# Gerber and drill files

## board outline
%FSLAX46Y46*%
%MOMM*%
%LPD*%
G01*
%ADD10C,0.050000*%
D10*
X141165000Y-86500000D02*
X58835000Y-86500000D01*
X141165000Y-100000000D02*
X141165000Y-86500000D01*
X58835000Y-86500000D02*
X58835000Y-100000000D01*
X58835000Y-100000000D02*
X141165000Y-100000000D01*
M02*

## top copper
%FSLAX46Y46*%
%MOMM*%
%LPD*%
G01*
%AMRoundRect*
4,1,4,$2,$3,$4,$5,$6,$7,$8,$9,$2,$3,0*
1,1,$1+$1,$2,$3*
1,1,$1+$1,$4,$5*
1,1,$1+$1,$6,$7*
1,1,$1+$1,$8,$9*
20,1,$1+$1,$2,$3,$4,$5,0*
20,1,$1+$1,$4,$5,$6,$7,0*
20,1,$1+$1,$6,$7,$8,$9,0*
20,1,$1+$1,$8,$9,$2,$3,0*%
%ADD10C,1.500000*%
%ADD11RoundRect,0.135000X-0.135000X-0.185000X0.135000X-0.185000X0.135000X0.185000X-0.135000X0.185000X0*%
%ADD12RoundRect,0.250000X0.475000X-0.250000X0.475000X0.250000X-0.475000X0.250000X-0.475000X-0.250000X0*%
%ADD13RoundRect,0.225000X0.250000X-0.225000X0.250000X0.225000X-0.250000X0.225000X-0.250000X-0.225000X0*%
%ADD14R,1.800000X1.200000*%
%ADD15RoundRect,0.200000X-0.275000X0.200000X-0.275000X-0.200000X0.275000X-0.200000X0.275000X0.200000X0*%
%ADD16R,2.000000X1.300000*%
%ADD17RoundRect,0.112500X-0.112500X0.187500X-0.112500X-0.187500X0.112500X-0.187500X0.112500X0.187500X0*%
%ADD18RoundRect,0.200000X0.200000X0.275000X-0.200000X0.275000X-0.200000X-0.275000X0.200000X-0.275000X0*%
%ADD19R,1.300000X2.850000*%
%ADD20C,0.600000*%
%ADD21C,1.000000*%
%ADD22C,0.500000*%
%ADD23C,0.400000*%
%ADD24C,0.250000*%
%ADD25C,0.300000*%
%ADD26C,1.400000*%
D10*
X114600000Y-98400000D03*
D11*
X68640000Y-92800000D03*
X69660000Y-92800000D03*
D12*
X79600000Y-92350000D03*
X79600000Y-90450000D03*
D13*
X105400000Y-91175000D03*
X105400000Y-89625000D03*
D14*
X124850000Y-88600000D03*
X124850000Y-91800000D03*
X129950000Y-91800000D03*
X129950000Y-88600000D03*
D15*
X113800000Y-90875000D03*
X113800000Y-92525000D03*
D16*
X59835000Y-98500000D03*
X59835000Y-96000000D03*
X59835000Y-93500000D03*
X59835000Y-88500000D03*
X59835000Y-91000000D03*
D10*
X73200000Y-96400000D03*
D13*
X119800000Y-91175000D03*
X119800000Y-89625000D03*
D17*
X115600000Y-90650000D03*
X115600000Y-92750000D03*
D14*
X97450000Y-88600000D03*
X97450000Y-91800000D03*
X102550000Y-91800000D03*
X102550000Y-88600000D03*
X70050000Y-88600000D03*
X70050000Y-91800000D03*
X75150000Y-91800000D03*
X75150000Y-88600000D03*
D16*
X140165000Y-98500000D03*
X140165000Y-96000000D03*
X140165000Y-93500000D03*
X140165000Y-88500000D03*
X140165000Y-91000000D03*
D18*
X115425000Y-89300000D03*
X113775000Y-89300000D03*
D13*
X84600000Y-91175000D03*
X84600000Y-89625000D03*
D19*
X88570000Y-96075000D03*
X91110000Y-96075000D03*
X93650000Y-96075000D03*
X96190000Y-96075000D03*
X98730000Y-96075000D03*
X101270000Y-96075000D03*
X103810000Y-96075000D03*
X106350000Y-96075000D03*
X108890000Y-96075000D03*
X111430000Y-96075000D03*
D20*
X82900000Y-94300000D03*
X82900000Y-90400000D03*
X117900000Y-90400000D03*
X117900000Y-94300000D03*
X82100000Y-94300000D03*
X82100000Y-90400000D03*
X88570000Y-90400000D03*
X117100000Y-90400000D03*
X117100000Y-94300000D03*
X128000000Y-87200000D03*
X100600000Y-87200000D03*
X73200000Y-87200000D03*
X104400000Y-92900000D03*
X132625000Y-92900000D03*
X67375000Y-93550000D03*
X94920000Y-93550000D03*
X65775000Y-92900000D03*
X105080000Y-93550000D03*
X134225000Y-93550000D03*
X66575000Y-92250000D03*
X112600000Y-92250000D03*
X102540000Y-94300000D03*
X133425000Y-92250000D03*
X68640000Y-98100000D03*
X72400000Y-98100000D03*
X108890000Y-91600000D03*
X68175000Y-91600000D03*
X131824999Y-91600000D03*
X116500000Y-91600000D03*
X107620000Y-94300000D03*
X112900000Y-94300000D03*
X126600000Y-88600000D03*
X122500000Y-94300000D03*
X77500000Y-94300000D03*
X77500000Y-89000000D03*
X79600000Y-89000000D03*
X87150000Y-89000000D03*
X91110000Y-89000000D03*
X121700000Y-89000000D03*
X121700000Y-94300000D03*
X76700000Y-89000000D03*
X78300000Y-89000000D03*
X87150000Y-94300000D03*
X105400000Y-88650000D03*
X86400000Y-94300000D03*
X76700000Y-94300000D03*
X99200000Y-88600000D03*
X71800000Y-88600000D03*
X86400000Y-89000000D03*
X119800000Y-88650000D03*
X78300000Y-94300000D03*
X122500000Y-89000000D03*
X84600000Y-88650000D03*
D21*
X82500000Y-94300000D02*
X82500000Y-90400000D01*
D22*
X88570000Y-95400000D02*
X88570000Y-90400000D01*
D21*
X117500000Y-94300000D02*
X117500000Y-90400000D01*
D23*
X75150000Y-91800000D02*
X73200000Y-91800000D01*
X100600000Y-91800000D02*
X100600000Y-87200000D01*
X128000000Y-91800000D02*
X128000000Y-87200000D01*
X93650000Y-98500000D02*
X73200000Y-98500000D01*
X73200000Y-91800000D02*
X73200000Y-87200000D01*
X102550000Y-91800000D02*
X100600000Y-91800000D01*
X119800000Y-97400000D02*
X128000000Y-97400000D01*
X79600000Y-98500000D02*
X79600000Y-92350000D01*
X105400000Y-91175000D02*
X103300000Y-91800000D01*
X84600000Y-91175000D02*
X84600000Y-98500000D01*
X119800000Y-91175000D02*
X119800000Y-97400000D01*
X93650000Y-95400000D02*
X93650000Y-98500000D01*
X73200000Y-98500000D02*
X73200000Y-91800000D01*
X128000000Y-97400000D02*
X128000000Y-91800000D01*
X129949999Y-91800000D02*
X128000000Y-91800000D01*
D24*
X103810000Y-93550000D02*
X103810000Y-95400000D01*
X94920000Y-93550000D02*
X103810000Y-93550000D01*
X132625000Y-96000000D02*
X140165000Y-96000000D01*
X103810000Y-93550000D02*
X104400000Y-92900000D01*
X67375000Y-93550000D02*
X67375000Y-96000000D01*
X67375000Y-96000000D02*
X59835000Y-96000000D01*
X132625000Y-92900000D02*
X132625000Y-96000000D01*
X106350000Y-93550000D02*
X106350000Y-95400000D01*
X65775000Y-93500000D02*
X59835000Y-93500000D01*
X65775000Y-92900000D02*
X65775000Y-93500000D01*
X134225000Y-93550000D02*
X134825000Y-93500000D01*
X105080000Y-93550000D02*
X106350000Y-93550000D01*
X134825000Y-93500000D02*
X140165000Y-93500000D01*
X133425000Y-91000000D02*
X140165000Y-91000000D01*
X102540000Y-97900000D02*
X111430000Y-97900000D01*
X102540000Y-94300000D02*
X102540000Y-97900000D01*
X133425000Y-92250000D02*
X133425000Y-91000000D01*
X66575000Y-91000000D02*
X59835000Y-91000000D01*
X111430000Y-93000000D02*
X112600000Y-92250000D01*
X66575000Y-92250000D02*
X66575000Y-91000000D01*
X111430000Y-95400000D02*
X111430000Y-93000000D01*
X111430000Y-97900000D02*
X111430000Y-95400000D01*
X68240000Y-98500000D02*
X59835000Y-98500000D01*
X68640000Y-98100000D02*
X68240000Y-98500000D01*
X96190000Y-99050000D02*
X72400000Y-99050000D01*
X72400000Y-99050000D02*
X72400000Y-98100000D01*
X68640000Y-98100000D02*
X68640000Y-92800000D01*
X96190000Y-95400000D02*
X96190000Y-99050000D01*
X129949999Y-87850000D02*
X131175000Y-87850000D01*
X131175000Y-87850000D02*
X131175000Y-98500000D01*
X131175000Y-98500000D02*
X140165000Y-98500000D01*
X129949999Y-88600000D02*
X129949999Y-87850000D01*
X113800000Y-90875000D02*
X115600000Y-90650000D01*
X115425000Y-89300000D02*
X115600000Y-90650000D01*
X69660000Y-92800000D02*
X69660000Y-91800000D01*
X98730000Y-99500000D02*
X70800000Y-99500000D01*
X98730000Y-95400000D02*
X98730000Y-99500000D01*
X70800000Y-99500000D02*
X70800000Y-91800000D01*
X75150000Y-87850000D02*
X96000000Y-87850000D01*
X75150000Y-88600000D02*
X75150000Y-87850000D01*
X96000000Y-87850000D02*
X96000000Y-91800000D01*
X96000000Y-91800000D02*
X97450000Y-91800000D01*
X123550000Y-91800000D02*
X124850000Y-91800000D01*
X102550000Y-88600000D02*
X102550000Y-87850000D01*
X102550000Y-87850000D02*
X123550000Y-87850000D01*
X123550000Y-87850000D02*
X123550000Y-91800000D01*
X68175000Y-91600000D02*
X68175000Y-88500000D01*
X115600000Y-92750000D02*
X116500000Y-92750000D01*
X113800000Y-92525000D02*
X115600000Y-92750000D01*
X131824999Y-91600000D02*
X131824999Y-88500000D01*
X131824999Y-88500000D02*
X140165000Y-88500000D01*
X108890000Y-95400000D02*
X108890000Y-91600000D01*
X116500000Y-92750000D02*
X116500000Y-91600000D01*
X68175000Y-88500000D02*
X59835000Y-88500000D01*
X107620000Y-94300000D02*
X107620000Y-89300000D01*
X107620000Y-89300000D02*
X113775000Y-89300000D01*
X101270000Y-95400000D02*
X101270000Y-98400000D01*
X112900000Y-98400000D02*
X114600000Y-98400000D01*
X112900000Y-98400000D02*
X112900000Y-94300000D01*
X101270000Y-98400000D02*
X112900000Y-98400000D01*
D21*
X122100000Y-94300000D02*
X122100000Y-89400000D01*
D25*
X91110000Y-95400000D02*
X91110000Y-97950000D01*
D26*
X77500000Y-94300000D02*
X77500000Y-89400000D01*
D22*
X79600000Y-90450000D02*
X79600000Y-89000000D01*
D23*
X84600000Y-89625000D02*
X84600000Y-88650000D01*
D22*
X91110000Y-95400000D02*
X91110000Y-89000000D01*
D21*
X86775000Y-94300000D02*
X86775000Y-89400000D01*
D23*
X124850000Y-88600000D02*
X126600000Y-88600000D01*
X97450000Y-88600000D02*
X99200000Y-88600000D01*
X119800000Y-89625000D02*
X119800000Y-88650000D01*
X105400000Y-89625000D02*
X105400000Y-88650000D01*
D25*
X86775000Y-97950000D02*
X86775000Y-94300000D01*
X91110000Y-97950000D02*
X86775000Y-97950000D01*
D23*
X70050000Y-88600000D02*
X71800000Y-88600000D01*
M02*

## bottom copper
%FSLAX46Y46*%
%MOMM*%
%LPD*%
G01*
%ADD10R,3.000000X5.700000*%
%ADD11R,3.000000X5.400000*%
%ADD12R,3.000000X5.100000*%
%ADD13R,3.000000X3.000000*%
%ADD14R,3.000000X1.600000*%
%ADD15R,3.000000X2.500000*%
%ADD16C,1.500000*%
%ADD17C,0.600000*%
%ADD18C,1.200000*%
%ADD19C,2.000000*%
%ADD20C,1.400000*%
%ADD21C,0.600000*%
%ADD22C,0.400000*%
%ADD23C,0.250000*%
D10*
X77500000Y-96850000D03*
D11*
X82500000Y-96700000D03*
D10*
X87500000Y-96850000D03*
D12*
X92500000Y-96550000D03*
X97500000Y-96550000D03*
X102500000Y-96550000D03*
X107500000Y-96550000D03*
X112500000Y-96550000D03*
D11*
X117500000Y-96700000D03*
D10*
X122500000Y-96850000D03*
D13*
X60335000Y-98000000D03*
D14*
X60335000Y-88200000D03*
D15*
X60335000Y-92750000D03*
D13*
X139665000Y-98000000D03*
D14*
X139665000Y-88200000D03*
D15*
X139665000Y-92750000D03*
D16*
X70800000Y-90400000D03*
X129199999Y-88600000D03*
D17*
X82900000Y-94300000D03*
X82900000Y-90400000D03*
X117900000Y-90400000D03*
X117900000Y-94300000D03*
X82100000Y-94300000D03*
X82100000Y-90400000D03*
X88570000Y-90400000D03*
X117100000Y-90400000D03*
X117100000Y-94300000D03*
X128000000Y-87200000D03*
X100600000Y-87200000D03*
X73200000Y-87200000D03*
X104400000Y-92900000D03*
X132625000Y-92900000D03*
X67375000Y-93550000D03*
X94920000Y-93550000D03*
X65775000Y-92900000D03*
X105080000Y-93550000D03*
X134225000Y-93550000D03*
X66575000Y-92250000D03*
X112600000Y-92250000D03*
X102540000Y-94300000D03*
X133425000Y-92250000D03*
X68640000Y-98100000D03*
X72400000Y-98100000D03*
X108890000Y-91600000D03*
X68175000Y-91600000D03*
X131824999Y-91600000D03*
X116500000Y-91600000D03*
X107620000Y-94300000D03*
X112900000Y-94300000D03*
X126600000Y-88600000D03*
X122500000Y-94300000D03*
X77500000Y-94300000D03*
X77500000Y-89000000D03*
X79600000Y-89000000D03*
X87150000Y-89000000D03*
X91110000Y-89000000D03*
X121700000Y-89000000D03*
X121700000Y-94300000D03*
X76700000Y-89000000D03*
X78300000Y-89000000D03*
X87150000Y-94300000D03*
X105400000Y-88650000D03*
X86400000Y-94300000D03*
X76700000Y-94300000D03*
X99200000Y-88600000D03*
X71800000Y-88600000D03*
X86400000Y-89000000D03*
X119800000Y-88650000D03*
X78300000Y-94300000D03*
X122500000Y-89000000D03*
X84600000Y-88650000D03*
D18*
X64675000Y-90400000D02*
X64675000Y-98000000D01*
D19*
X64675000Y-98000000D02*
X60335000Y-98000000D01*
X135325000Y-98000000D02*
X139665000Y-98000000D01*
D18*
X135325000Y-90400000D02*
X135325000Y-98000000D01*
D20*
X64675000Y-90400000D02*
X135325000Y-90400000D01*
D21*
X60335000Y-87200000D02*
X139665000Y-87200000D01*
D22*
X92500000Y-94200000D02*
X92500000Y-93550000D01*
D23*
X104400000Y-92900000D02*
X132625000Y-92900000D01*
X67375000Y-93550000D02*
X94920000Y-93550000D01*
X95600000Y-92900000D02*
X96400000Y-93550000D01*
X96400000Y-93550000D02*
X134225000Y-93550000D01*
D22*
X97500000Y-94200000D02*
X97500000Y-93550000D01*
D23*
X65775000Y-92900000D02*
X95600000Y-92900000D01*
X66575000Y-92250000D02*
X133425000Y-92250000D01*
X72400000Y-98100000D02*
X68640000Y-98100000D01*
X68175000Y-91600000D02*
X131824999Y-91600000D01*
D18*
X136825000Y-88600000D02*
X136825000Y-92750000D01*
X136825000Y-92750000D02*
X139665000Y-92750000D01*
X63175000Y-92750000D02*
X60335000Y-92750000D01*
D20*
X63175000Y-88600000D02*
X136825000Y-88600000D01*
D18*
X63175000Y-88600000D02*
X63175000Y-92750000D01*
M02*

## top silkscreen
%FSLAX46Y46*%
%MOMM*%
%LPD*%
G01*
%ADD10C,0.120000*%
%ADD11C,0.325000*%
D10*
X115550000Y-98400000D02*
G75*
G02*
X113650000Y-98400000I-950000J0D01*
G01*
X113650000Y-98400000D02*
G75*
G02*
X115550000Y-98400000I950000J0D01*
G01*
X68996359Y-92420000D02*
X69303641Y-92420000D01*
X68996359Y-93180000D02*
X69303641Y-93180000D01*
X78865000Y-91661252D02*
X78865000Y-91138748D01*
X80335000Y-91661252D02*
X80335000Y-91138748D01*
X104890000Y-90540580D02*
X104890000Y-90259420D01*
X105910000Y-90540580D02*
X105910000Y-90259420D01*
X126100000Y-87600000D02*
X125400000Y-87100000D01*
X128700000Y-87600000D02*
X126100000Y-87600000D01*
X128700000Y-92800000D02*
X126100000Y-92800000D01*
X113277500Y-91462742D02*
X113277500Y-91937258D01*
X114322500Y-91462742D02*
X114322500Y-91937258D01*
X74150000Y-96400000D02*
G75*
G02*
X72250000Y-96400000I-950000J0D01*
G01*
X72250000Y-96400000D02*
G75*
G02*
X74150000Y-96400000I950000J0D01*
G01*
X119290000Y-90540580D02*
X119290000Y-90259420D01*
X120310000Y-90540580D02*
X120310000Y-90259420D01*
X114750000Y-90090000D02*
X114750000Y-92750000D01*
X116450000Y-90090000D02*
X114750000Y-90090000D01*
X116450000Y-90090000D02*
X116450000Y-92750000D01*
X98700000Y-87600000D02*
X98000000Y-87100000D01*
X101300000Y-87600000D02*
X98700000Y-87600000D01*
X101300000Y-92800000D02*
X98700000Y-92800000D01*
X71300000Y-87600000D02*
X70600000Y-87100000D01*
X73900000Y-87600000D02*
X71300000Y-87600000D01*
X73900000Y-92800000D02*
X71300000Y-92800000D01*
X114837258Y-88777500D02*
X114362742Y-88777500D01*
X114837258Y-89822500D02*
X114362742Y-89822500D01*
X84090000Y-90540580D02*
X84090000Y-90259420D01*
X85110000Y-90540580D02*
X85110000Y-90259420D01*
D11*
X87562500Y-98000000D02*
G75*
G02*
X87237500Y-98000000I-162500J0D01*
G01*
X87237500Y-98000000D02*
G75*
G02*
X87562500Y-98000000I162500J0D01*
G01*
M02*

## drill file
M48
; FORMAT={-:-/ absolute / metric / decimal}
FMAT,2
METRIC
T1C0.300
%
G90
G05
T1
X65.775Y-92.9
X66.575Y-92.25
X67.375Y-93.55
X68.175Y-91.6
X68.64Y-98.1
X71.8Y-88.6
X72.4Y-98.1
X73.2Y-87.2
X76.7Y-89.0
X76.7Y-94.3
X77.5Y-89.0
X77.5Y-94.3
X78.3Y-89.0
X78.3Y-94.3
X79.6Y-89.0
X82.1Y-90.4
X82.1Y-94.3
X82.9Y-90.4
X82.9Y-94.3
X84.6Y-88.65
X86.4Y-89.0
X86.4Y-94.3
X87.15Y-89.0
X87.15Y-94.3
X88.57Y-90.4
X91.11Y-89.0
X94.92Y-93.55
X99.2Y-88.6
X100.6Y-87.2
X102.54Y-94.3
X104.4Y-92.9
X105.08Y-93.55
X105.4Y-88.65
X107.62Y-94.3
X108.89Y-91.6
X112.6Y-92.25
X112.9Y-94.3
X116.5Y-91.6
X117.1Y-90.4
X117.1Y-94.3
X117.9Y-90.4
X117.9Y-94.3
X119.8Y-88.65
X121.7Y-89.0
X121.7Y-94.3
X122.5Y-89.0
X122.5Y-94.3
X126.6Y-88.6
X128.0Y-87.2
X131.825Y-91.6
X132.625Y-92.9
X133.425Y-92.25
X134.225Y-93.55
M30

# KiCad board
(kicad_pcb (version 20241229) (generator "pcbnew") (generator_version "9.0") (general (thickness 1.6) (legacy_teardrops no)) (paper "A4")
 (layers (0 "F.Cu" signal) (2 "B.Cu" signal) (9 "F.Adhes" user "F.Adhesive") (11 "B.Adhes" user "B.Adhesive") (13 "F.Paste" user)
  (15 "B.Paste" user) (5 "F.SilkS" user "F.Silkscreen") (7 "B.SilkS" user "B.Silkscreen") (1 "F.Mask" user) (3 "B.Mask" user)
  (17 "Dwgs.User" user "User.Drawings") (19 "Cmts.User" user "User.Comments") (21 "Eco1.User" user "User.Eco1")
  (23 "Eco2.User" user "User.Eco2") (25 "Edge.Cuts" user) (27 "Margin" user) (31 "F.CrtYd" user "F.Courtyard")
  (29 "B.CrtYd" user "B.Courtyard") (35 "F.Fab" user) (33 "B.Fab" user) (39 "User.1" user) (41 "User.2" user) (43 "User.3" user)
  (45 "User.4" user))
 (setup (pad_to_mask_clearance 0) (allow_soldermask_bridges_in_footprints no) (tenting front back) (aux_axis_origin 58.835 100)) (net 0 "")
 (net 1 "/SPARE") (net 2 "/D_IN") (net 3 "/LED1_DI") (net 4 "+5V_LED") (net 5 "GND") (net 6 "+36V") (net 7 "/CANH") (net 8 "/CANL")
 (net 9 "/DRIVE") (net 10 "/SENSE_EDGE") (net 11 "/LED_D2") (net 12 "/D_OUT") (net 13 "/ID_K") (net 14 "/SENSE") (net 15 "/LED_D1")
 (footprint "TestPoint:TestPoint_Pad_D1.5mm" (layer "F.Cu") (at 114.6 98.4)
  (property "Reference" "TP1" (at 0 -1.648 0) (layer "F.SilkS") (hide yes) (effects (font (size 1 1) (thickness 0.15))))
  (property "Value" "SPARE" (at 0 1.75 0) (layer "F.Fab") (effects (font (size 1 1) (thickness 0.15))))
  (fp_circle (center 0 0) (end 0 0.95) (stroke (width 0.12) (type solid)) (fill no) (layer "F.SilkS"))
  (pad "1" smd circle (at 0 0) (size 1.5 1.5) (layers "F.Cu" "F.Mask") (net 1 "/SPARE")))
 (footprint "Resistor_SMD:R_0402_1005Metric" (layer "F.Cu") (at 69.15 92.8)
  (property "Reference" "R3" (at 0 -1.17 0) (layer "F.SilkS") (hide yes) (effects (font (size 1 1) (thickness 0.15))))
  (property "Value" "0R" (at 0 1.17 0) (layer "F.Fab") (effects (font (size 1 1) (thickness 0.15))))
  (fp_line (start -0.153641 -0.38) (end 0.153641 -0.38) (stroke (width 0.12) (type solid)) (layer "F.SilkS"))
  (fp_line (start -0.153641 0.38) (end 0.153641 0.38) (stroke (width 0.12) (type solid)) (layer "F.SilkS"))
  (pad "1" smd roundrect (at -0.51 0) (size 0.54 0.64) (layers "F.Cu" "F.Mask" "F.Paste") (roundrect_rratio 0.25) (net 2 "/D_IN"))
  (pad "2" smd roundrect (at 0.51 0) (size 0.54 0.64) (layers "F.Cu" "F.Mask" "F.Paste") (roundrect_rratio 0.25) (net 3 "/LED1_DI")))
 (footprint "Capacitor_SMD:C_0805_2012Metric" (layer "F.Cu") (at 79.6 91.4 90)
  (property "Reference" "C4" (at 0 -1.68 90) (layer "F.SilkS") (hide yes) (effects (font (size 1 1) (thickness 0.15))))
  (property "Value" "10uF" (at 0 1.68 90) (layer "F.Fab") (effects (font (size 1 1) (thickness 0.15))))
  (fp_line (start -0.261252 -0.735) (end 0.261252 -0.735) (stroke (width 0.12) (type solid)) (layer "F.SilkS"))
  (fp_line (start -0.261252 0.735) (end 0.261252 0.735) (stroke (width 0.12) (type solid)) (layer "F.SilkS"))
  (pad "1" smd roundrect (at -0.95 0 90) (size 1 1.45) (layers "F.Cu" "F.Mask" "F.Paste") (roundrect_rratio 0.25) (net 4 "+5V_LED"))
  (pad "2" smd roundrect (at 0.95 0 90) (size 1 1.45) (layers "F.Cu" "F.Mask" "F.Paste") (roundrect_rratio 0.25) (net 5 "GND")))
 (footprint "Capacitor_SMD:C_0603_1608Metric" (layer "F.Cu") (at 105.4 90.4 90)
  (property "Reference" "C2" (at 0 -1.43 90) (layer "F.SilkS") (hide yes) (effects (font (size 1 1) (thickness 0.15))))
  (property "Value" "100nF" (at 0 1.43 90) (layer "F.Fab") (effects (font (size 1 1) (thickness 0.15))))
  (fp_line (start -0.14058 -0.51) (end 0.14058 -0.51) (stroke (width 0.12) (type solid)) (layer "F.SilkS"))
  (fp_line (start -0.14058 0.51) (end 0.14058 0.51) (stroke (width 0.12) (type solid)) (layer "F.SilkS"))
  (pad "1" smd roundrect (at -0.775 0 90) (size 0.9 0.95) (layers "F.Cu" "F.Mask" "F.Paste") (roundrect_rratio 0.25) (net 4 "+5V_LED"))
  (pad "2" smd roundrect (at 0.775 0 90) (size 0.9 0.95) (layers "F.Cu" "F.Mask" "F.Paste") (roundrect_rratio 0.25) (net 5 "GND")))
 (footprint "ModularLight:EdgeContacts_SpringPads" (layer "F.Cu") (at 100 100)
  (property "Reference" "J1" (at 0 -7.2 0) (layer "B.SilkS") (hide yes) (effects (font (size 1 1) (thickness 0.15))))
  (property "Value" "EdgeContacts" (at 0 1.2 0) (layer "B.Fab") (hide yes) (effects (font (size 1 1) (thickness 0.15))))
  (pad "X1" smd rect (at -22.5 -3.15) (size 3 5.7) (layers "B.Cu" "B.Mask") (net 5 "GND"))
  (pad "X2" smd rect (at -17.5 -3.3) (size 3 5.4) (layers "B.Cu" "B.Mask") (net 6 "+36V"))
  (pad "X3" smd rect (at -12.5 -3.15) (size 3 5.7) (layers "B.Cu" "B.Mask") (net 5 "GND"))
  (pad "X4" smd rect (at -7.5 -3.45) (size 3 5.1) (layers "B.Cu" "B.Mask") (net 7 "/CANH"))
  (pad "X5" smd rect (at -2.5 -3.45) (size 3 5.1) (layers "B.Cu" "B.Mask") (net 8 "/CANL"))
  (pad "X6" smd rect (at 2.5 -3.45) (size 3 5.1) (layers "B.Cu" "B.Mask") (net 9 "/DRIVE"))
  (pad "X7" smd rect (at 7.5 -3.45) (size 3 5.1) (layers "B.Cu" "B.Mask") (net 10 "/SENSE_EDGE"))
  (pad "X8" smd rect (at 12.5 -3.45) (size 3 5.1) (layers "B.Cu" "B.Mask") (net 1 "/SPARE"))
  (pad "X9" smd rect (at 17.5 -3.3) (size 3 5.4) (layers "B.Cu" "B.Mask") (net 6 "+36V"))
  (pad "X10" smd rect (at 22.5 -3.15) (size 3 5.7) (layers "B.Cu" "B.Mask") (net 5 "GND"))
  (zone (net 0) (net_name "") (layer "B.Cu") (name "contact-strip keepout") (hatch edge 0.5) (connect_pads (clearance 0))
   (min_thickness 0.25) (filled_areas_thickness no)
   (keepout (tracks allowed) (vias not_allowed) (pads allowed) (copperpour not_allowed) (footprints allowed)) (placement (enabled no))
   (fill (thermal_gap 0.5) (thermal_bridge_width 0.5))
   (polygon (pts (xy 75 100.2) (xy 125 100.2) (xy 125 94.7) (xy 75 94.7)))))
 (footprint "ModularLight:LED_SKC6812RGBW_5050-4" (layer "F.Cu") (at 127.4 90.2 180)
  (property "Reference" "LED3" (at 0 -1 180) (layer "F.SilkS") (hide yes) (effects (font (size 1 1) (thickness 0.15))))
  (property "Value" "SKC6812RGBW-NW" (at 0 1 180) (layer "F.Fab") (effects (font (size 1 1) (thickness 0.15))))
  (fp_line (start 1.3 2.6) (end 2 3.1) (stroke (width 0.12) (type solid)) (layer "F.SilkS"))
  (fp_line (start -1.3 2.6) (end 1.3 2.6) (stroke (width 0.12) (type solid)) (layer "F.SilkS"))
  (fp_line (start -1.3 -2.6) (end 1.3 -2.6) (stroke (width 0.12) (type solid)) (layer "F.SilkS"))
  (pad "1" smd rect (at 2.55 1.6 180) (size 1.8 1.2) (layers "F.Cu" "F.Mask" "F.Paste") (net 5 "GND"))
  (pad "2" smd rect (at 2.55 -1.6 180) (size 1.8 1.2) (layers "F.Cu" "F.Mask" "F.Paste") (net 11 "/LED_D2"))
  (pad "3" smd rect (at -2.55 -1.6 180) (size 1.8 1.2) (layers "F.Cu" "F.Mask" "F.Paste") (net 4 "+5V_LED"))
  (pad "4" smd rect (at -2.55 1.6 180) (size 1.8 1.2) (layers "F.Cu" "F.Mask" "F.Paste") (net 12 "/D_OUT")))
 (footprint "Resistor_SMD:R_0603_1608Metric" (layer "F.Cu") (at 113.8 91.7 -90)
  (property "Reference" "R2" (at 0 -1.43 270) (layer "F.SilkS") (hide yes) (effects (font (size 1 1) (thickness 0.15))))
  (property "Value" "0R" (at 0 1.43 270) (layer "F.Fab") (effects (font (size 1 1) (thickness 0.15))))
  (fp_line (start -0.237258 0.5225) (end 0.237258 0.5225) (stroke (width 0.12) (type solid)) (layer "F.SilkS"))
  (fp_line (start -0.237258 -0.5225) (end 0.237258 -0.5225) (stroke (width 0.12) (type solid)) (layer "F.SilkS"))
  (pad "1" smd roundrect (at -0.825 0 270) (size 0.8 0.95) (layers "F.Cu" "F.Mask" "F.Paste") (roundrect_rratio 0.25) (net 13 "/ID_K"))
  (pad "2" smd roundrect (at 0.825 0 270) (size 0.8 0.95) (layers "F.Cu" "F.Mask" "F.Paste") (roundrect_rratio 0.25) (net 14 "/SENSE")))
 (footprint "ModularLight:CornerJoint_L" (layer "F.Cu") (at 58.835 100)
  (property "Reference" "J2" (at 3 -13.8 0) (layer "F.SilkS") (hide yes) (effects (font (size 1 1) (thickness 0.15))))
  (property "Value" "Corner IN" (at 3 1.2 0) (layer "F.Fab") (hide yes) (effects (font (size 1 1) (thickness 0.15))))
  (pad "1" smd rect (at 1 -1.5) (size 2 1.3) (layers "F.Cu" "F.Mask" "F.Paste") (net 2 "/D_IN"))
  (pad "2" smd rect (at 1 -4) (size 2 1.3) (layers "F.Cu" "F.Mask" "F.Paste") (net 7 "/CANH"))
  (pad "3" smd rect (at 1 -6.5) (size 2 1.3) (layers "F.Cu" "F.Mask" "F.Paste") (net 8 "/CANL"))
  (pad "4" smd rect (at 1 -11.5) (size 2 1.3) (layers "F.Cu" "F.Mask" "F.Paste") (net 14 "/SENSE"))
  (pad "5" smd rect (at 1 -9) (size 2 1.3) (layers "F.Cu" "F.Mask" "F.Paste") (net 9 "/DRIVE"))
  (pad "6" smd rect (at 1.5 -2) (size 3 3) (layers "B.Cu" "B.Mask") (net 6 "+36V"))
  (pad "7" smd rect (at 1.5 -11.8) (size 3 1.6) (layers "B.Cu" "B.Mask") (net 4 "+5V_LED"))
  (pad "8" smd rect (at 1.5 -7.25) (size 3 2.5) (layers "B.Cu" "B.Mask") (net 5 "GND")))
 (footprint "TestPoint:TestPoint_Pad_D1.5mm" (layer "F.Cu") (at 73.2 96.4)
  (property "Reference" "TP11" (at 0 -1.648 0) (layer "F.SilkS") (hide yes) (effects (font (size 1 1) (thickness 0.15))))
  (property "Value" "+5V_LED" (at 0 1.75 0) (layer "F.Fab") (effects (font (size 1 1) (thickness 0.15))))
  (fp_circle (center 0 0) (end 0 0.95) (stroke (width 0.12) (type solid)) (fill no) (layer "F.SilkS"))
  (pad "1" smd circle (at 0 0) (size 1.5 1.5) (layers "F.Cu" "F.Mask") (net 4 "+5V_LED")))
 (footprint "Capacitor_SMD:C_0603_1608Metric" (layer "F.Cu") (at 119.8 90.4 90)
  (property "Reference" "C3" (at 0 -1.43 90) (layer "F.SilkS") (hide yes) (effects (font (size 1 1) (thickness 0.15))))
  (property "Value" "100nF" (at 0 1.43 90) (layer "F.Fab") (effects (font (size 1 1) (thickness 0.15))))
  (fp_line (start -0.14058 -0.51) (end 0.14058 -0.51) (stroke (width 0.12) (type solid)) (layer "F.SilkS"))
  (fp_line (start -0.14058 0.51) (end 0.14058 0.51) (stroke (width 0.12) (type solid)) (layer "F.SilkS"))
  (pad "1" smd roundrect (at -0.775 0 90) (size 0.9 0.95) (layers "F.Cu" "F.Mask" "F.Paste") (roundrect_rratio 0.25) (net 4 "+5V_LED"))
  (pad "2" smd roundrect (at 0.775 0 90) (size 0.9 0.95) (layers "F.Cu" "F.Mask" "F.Paste") (roundrect_rratio 0.25) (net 5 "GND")))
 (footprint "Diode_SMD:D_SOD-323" (layer "F.Cu") (at 115.6 91.7 -90)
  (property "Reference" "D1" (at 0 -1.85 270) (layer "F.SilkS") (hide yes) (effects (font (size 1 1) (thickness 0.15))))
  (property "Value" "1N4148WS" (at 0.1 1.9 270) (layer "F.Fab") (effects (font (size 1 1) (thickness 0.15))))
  (fp_line (start -1.61 0.85) (end 1.05 0.85) (stroke (width 0.12) (type solid)) (layer "F.SilkS"))
  (fp_line (start -1.61 -0.85) (end -1.61 0.85) (stroke (width 0.12) (type solid)) (layer "F.SilkS"))
  (fp_line (start -1.61 -0.85) (end 1.05 -0.85) (stroke (width 0.12) (type solid)) (layer "F.SilkS"))
  (pad "1" smd roundrect (at -1.05 0 270) (size 0.6 0.45) (layers "F.Cu" "F.Mask" "F.Paste") (roundrect_rratio 0.25) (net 13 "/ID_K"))
  (pad "2" smd roundrect (at 1.05 0 270) (size 0.6 0.45) (layers "F.Cu" "F.Mask" "F.Paste") (roundrect_rratio 0.25) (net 14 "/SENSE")))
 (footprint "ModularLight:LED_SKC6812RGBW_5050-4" (layer "F.Cu") (at 100 90.2 180)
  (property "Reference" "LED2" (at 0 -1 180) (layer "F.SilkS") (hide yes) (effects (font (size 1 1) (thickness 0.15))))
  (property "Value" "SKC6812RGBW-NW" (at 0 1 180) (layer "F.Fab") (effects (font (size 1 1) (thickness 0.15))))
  (fp_line (start 1.3 2.6) (end 2 3.1) (stroke (width 0.12) (type solid)) (layer "F.SilkS"))
  (fp_line (start -1.3 2.6) (end 1.3 2.6) (stroke (width 0.12) (type solid)) (layer "F.SilkS"))
  (fp_line (start -1.3 -2.6) (end 1.3 -2.6) (stroke (width 0.12) (type solid)) (layer "F.SilkS"))
  (pad "1" smd rect (at 2.55 1.6 180) (size 1.8 1.2) (layers "F.Cu" "F.Mask" "F.Paste") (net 5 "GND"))
  (pad "2" smd rect (at 2.55 -1.6 180) (size 1.8 1.2) (layers "F.Cu" "F.Mask" "F.Paste") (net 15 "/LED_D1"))
  (pad "3" smd rect (at -2.55 -1.6 180) (size 1.8 1.2) (layers "F.Cu" "F.Mask" "F.Paste") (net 4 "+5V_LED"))
  (pad "4" smd rect (at -2.55 1.6 180) (size 1.8 1.2) (layers "F.Cu" "F.Mask" "F.Paste") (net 11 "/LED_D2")))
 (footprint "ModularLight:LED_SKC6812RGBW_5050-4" (layer "F.Cu") (at 72.6 90.2 180)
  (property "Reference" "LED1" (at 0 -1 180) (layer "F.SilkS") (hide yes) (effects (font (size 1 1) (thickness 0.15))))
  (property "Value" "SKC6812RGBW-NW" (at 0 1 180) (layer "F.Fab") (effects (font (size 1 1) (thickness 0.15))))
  (fp_line (start 1.3 2.6) (end 2 3.1) (stroke (width 0.12) (type solid)) (layer "F.SilkS"))
  (fp_line (start -1.3 2.6) (end 1.3 2.6) (stroke (width 0.12) (type solid)) (layer "F.SilkS"))
  (fp_line (start -1.3 -2.6) (end 1.3 -2.6) (stroke (width 0.12) (type solid)) (layer "F.SilkS"))
  (pad "1" smd rect (at 2.55 1.6 180) (size 1.8 1.2) (layers "F.Cu" "F.Mask" "F.Paste") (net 5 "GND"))
  (pad "2" smd rect (at 2.55 -1.6 180) (size 1.8 1.2) (layers "F.Cu" "F.Mask" "F.Paste") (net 3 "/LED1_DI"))
  (pad "3" smd rect (at -2.55 -1.6 180) (size 1.8 1.2) (layers "F.Cu" "F.Mask" "F.Paste") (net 4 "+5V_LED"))
  (pad "4" smd rect (at -2.55 1.6 180) (size 1.8 1.2) (layers "F.Cu" "F.Mask" "F.Paste") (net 15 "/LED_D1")))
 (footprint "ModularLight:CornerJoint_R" (layer "F.Cu") (at 141.165 100)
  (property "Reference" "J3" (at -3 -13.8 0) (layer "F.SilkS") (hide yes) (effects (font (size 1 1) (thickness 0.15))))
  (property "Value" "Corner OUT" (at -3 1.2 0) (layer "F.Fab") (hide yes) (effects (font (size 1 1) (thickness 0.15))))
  (pad "1" smd rect (at -1 -1.5) (size 2 1.3) (layers "F.Cu" "F.Mask" "F.Paste") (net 12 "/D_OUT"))
  (pad "2" smd rect (at -1 -4) (size 2 1.3) (layers "F.Cu" "F.Mask" "F.Paste") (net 7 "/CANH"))
  (pad "3" smd rect (at -1 -6.5) (size 2 1.3) (layers "F.Cu" "F.Mask" "F.Paste") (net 8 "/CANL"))
  (pad "4" smd rect (at -1 -11.5) (size 2 1.3) (layers "F.Cu" "F.Mask" "F.Paste") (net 14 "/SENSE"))
  (pad "5" smd rect (at -1 -9) (size 2 1.3) (layers "F.Cu" "F.Mask" "F.Paste") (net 9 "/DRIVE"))
  (pad "6" smd rect (at -1.5 -2) (size 3 3) (layers "B.Cu" "B.Mask") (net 6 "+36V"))
  (pad "7" smd rect (at -1.5 -11.8) (size 3 1.6) (layers "B.Cu" "B.Mask") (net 4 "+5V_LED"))
  (pad "8" smd rect (at -1.5 -7.25) (size 3 2.5) (layers "B.Cu" "B.Mask") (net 5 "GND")))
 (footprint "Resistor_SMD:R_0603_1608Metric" (layer "F.Cu") (at 114.6 89.3 180)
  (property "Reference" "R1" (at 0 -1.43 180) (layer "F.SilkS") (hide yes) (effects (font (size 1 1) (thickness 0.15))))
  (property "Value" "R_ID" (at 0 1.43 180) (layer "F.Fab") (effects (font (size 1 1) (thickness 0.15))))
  (fp_line (start -0.237258 0.5225) (end 0.237258 0.5225) (stroke (width 0.12) (type solid)) (layer "F.SilkS"))
  (fp_line (start -0.237258 -0.5225) (end 0.237258 -0.5225) (stroke (width 0.12) (type solid)) (layer "F.SilkS"))
  (pad "1" smd roundrect (at -0.825 0 180) (size 0.8 0.95) (layers "F.Cu" "F.Mask" "F.Paste") (roundrect_rratio 0.25) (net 13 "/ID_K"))
  (pad "2" smd roundrect (at 0.825 0 180) (size 0.8 0.95) (layers "F.Cu" "F.Mask" "F.Paste") (roundrect_rratio 0.25) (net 10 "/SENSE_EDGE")))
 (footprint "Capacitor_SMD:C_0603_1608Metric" (layer "F.Cu") (at 84.6 90.4 90)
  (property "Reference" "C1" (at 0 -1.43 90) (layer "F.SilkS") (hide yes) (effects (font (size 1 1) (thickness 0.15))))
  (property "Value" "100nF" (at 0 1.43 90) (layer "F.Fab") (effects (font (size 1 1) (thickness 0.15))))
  (fp_line (start -0.14058 -0.51) (end 0.14058 -0.51) (stroke (width 0.12) (type solid)) (layer "F.SilkS"))
  (fp_line (start -0.14058 0.51) (end 0.14058 0.51) (stroke (width 0.12) (type solid)) (layer "F.SilkS"))
  (pad "1" smd roundrect (at -0.775 0 90) (size 0.9 0.95) (layers "F.Cu" "F.Mask" "F.Paste") (roundrect_rratio 0.25) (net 4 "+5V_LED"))
  (pad "2" smd roundrect (at 0.775 0 90) (size 0.9 0.95) (layers "F.Cu" "F.Mask" "F.Paste") (roundrect_rratio 0.25) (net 5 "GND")))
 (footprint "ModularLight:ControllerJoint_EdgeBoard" (layer "F.Cu") (at 100 94.75)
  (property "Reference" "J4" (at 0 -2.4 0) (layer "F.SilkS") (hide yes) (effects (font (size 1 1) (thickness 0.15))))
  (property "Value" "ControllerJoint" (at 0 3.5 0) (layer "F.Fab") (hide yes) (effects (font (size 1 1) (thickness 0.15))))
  (fp_circle (center -12.6 3.25) (end -12.35 3.25) (stroke (width 0.15) (type solid)) (fill yes) (layer "F.SilkS"))
  (pad "1" smd rect (at -11.43 1.325) (size 1.3 2.85) (layers "F.Cu" "F.Mask" "F.Paste") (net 6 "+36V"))
  (pad "2" smd rect (at -8.89 1.325) (size 1.3 2.85) (layers "F.Cu" "F.Mask" "F.Paste") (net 5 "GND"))
  (pad "3" smd rect (at -6.35 1.325) (size 1.3 2.85) (layers "F.Cu" "F.Mask" "F.Paste") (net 4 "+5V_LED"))
  (pad "4" smd rect (at -3.81 1.325) (size 1.3 2.85) (layers "F.Cu" "F.Mask" "F.Paste") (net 2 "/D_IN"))
  (pad "5" smd rect (at -1.27 1.325) (size 1.3 2.85) (layers "F.Cu" "F.Mask" "F.Paste") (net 3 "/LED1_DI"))
  (pad "6" smd rect (at 1.27 1.325) (size 1.3 2.85) (layers "F.Cu" "F.Mask" "F.Paste") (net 1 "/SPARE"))
  (pad "7" smd rect (at 3.81 1.325) (size 1.3 2.85) (layers "F.Cu" "F.Mask" "F.Paste") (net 7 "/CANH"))
  (pad "8" smd rect (at 6.35 1.325) (size 1.3 2.85) (layers "F.Cu" "F.Mask" "F.Paste") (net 8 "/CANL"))
  (pad "9" smd rect (at 8.89 1.325) (size 1.3 2.85) (layers "F.Cu" "F.Mask" "F.Paste") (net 14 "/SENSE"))
  (pad "10" smd rect (at 11.43 1.325) (size 1.3 2.85) (layers "F.Cu" "F.Mask" "F.Paste") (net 9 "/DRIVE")))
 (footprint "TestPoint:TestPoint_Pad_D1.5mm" (layer "B.Cu") (at 70.8 90.4 180)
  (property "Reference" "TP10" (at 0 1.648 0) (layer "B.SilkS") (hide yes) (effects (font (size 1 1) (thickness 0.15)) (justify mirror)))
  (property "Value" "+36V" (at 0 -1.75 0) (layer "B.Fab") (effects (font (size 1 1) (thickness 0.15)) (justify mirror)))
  (pad "1" smd circle (at 0 0 180) (size 1.5 1.5) (layers "B.Cu" "B.Mask") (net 6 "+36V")))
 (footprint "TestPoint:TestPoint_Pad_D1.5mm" (layer "B.Cu") (at 129.199999 88.6 180)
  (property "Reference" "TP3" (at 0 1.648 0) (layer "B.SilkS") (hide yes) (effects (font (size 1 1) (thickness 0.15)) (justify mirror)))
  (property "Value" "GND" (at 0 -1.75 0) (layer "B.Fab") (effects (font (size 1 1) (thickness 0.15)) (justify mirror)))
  (pad "1" smd circle (at 0 0 180) (size 1.5 1.5) (layers "B.Cu" "B.Mask") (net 5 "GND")))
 (gr_line (start 141.165 86.5) (end 58.835 86.5) (stroke (width 0.05) (type default)) (layer "Edge.Cuts"))
 (gr_line (start 141.165 100) (end 141.165 86.5) (stroke (width 0.05) (type default)) (layer "Edge.Cuts"))
 (gr_line (start 58.835 86.5) (end 58.835 100) (stroke (width 0.05) (type default)) (layer "Edge.Cuts"))
 (gr_line (start 58.835 100) (end 141.165 100) (stroke (width 0.05) (type default)) (layer "Edge.Cuts"))
 (segment (start 82.5 94.3) (end 82.5 90.4) (width 1) (locked yes) (layer "F.Cu") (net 6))
 (segment (start 88.57 95.4) (end 88.57 90.4) (width 0.5) (locked yes) (layer "F.Cu") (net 6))
 (segment (start 117.5 94.3) (end 117.5 90.4) (width 1) (locked yes) (layer "F.Cu") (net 6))
 (via (at 82.9 94.3) (size 0.6) (drill 0.3) (layers "F.Cu" "B.Cu") (locked yes) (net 6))
 (via (at 82.9 90.4) (size 0.6) (drill 0.3) (layers "F.Cu" "B.Cu") (locked yes) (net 6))
 (via (at 117.9 90.4) (size 0.6) (drill 0.3) (layers "F.Cu" "B.Cu") (locked yes) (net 6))
 (via (at 117.9 94.3) (size 0.6) (drill 0.3) (layers "F.Cu" "B.Cu") (locked yes) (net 6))
 (via (at 82.1 94.3) (size 0.6) (drill 0.3) (layers "F.Cu" "B.Cu") (locked yes) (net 6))
 (via (at 82.1 90.4) (size 0.6) (drill 0.3) (layers "F.Cu" "B.Cu") (locked yes) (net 6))
 (via (at 88.57 90.4) (size 0.6) (drill 0.3) (layers "F.Cu" "B.Cu") (locked yes) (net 6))
 (via (at 117.1 90.4) (size 0.6) (drill 0.3) (layers "F.Cu" "B.Cu") (locked yes) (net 6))
 (via (at 117.1 94.3) (size 0.6) (drill 0.3) (layers "F.Cu" "B.Cu") (locked yes) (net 6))
 (segment (start 64.675 90.4) (end 64.675 98) (width 1.2) (locked yes) (layer "B.Cu") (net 6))
 (segment (start 64.675 98) (end 60.335 98) (width 2) (locked yes) (layer "B.Cu") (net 6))
 (segment (start 135.325 98) (end 139.665 98) (width 2) (locked yes) (layer "B.Cu") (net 6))
 (segment (start 135.325 90.4) (end 135.325 98) (width 1.2) (locked yes) (layer "B.Cu") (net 6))
 (segment (start 64.675 90.4) (end 135.325 90.4) (width 1.4) (locked yes) (layer "B.Cu") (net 6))
 (segment (start 75.15 91.8) (end 73.2 91.8) (width 0.4) (locked yes) (layer "F.Cu") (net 4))
 (segment (start 100.6 91.8) (end 100.6 87.2) (width 0.4) (locked yes) (layer "F.Cu") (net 4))
 (segment (start 128 91.8) (end 128 87.2) (width 0.4) (locked yes) (layer "F.Cu") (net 4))
 (segment (start 93.65 98.5) (end 73.2 98.5) (width 0.4) (locked yes) (layer "F.Cu") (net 4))
 (segment (start 73.2 91.8) (end 73.2 87.2) (width 0.4) (locked yes) (layer "F.Cu") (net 4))
 (segment (start 102.55 91.8) (end 100.6 91.8) (width 0.4) (locked yes) (layer "F.Cu") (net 4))
 (segment (start 119.8 97.4) (end 128 97.4) (width 0.4) (locked yes) (layer "F.Cu") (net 4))
 (segment (start 79.6 98.5) (end 79.6 92.35) (width 0.4) (locked yes) (layer "F.Cu") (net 4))
 (segment (start 105.4 91.175) (end 103.3 91.8) (width 0.4) (locked yes) (layer "F.Cu") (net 4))
 (segment (start 84.6 91.175) (end 84.6 98.5) (width 0.4) (locked yes) (layer "F.Cu") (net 4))
 (segment (start 119.8 91.175) (end 119.8 97.4) (width 0.4) (locked yes) (layer "F.Cu") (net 4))
 (segment (start 93.65 95.4) (end 93.65 98.5) (width 0.4) (locked yes) (layer "F.Cu") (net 4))
 (segment (start 73.2 98.5) (end 73.2 91.8) (width 0.4) (locked yes) (layer "F.Cu") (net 4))
 (segment (start 128 97.4) (end 128 91.8) (width 0.4) (locked yes) (layer "F.Cu") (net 4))
 (segment (start 129.949999 91.8) (end 128 91.8) (width 0.4) (locked yes) (layer "F.Cu") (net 4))
 (via (at 128 87.2) (size 0.6) (drill 0.3) (layers "F.Cu" "B.Cu") (locked yes) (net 4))
 (via (at 100.6 87.2) (size 0.6) (drill 0.3) (layers "F.Cu" "B.Cu") (locked yes) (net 4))
 (via (at 73.2 87.2) (size 0.6) (drill 0.3) (layers "F.Cu" "B.Cu") (locked yes) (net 4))
 (segment (start 60.335 87.2) (end 139.665 87.2) (width 0.6) (locked yes) (layer "B.Cu") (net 4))
 (segment (start 103.81 93.55) (end 103.81 95.4) (width 0.25) (locked yes) (layer "F.Cu") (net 7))
 (segment (start 94.92 93.55) (end 103.81 93.55) (width 0.25) (locked yes) (layer "F.Cu") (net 7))
 (segment (start 132.625 96) (end 140.165 96) (width 0.25) (locked yes) (layer "F.Cu") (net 7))
 (segment (start 103.81 93.55) (end 104.4 92.9) (width 0.25) (locked yes) (layer "F.Cu") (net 7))
 (segment (start 67.375 93.55) (end 67.375 96) (width 0.25) (locked yes) (layer "F.Cu") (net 7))
 (segment (start 67.375 96) (end 59.835 96) (width 0.25) (locked yes) (layer "F.Cu") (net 7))
 (segment (start 132.625 92.9) (end 132.625 96) (width 0.25) (locked yes) (layer "F.Cu") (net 7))
 (via (at 104.4 92.9) (size 0.6) (drill 0.3) (layers "F.Cu" "B.Cu") (locked yes) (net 7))
 (via (at 132.625 92.9) (size 0.6) (drill 0.3) (layers "F.Cu" "B.Cu") (locked yes) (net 7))
 (via (at 67.375 93.55) (size 0.6) (drill 0.3) (layers "F.Cu" "B.Cu") (locked yes) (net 7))
 (via (at 94.92 93.55) (size 0.6) (drill 0.3) (layers "F.Cu" "B.Cu") (locked yes) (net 7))
 (segment (start 92.5 94.2) (end 92.5 93.55) (width 0.4) (locked yes) (layer "B.Cu") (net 7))
 (segment (start 104.4 92.9) (end 132.625 92.9) (width 0.25) (locked yes) (layer "B.Cu") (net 7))
 (segment (start 67.375 93.55) (end 94.92 93.55) (width 0.25) (locked yes) (layer "B.Cu") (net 7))
 (segment (start 106.35 93.55) (end 106.35 95.4) (width 0.25) (locked yes) (layer "F.Cu") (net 8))
 (segment (start 65.775 93.5) (end 59.835 93.5) (width 0.25) (locked yes) (layer "F.Cu") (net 8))
 (segment (start 65.775 92.9) (end 65.775 93.5) (width 0.25) (locked yes) (layer "F.Cu") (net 8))
 (segment (start 134.225 93.55) (end 134.825 93.5) (width 0.25) (locked yes) (layer "F.Cu") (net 8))
 (segment (start 105.08 93.55) (end 106.35 93.55) (width 0.25) (locked yes) (layer "F.Cu") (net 8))
 (segment (start 134.825 93.5) (end 140.165 93.5) (width 0.25) (locked yes) (layer "F.Cu") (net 8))
 (via (at 65.775 92.9) (size 0.6) (drill 0.3) (layers "F.Cu" "B.Cu") (locked yes) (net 8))
 (via (at 105.08 93.55) (size 0.6) (drill 0.3) (layers "F.Cu" "B.Cu") (locked yes) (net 8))
 (via (at 134.225 93.55) (size 0.6) (drill 0.3) (layers "F.Cu" "B.Cu") (locked yes) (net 8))
 (segment (start 95.6 92.9) (end 96.4 93.55) (width 0.25) (locked yes) (layer "B.Cu") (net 8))
 (segment (start 96.4 93.55) (end 134.225 93.55) (width 0.25) (locked yes) (layer "B.Cu") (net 8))
 (segment (start 97.5 94.2) (end 97.5 93.55) (width 0.4) (locked yes) (layer "B.Cu") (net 8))
 (segment (start 65.775 92.9) (end 95.6 92.9) (width 0.25) (locked yes) (layer "B.Cu") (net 8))
 (segment (start 133.425 91) (end 140.165 91) (width 0.25) (locked yes) (layer "F.Cu") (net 9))
 (segment (start 102.54 97.9) (end 111.43 97.9) (width 0.25) (locked yes) (layer "F.Cu") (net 9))
 (segment (start 102.54 94.3) (end 102.54 97.9) (width 0.25) (locked yes) (layer "F.Cu") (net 9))
 (segment (start 133.425 92.25) (end 133.425 91) (width 0.25) (locked yes) (layer "F.Cu") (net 9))
 (segment (start 66.575 91) (end 59.835 91) (width 0.25) (locked yes) (layer "F.Cu") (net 9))
 (segment (start 111.43 93) (end 112.6 92.25) (width 0.25) (locked yes) (layer "F.Cu") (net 9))
 (segment (start 66.575 92.25) (end 66.575 91) (width 0.25) (locked yes) (layer "F.Cu") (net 9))
 (segment (start 111.43 95.4) (end 111.43 93) (width 0.25) (locked yes) (layer "F.Cu") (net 9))
 (segment (start 111.43 97.9) (end 111.43 95.4) (width 0.25) (locked yes) (layer "F.Cu") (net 9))
 (via (at 66.575 92.25) (size 0.6) (drill 0.3) (layers "F.Cu" "B.Cu") (locked yes) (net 9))
 (via (at 112.6 92.25) (size 0.6) (drill 0.3) (layers "F.Cu" "B.Cu") (locked yes) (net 9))
 (via (at 102.54 94.3) (size 0.6) (drill 0.3) (layers "F.Cu" "B.Cu") (locked yes) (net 9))
 (via (at 133.425 92.25) (size 0.6) (drill 0.3) (layers "F.Cu" "B.Cu") (locked yes) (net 9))
 (segment (start 66.575 92.25) (end 133.425 92.25) (width 0.25) (locked yes) (layer "B.Cu") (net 9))
 (segment (start 68.24 98.5) (end 59.835 98.5) (width 0.25) (locked yes) (layer "F.Cu") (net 2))
 (segment (start 68.64 98.1) (end 68.24 98.5) (width 0.25) (locked yes) (layer "F.Cu") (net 2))
 (segment (start 96.19 99.05) (end 72.4 99.05) (width 0.25) (locked yes) (layer "F.Cu") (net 2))
 (segment (start 72.4 99.05) (end 72.4 98.1) (width 0.25) (locked yes) (layer "F.Cu") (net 2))
 (segment (start 68.64 98.1) (end 68.64 92.8) (width 0.25) (locked yes) (layer "F.Cu") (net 2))
 (segment (start 96.19 95.4) (end 96.19 99.05) (width 0.25) (locked yes) (layer "F.Cu") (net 2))
 (via (at 68.64 98.1) (size 0.6) (drill 0.3) (layers "F.Cu" "B.Cu") (locked yes) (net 2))
 (via (at 72.4 98.1) (size 0.6) (drill 0.3) (layers "F.Cu" "B.Cu") (locked yes) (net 2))
 (segment (start 72.4 98.1) (end 68.64 98.1) (width 0.25) (locked yes) (layer "B.Cu") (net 2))
 (segment (start 129.949999 87.85) (end 131.175 87.85) (width 0.25) (locked yes) (layer "F.Cu") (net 12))
 (segment (start 131.175 87.85) (end 131.175 98.5) (width 0.25) (locked yes) (layer "F.Cu") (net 12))
 (segment (start 131.175 98.5) (end 140.165 98.5) (width 0.25) (locked yes) (layer "F.Cu") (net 12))
 (segment (start 129.949999 88.6) (end 129.949999 87.85) (width 0.25) (locked yes) (layer "F.Cu") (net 12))
 (segment (start 113.8 90.875) (end 115.6 90.65) (width 0.25) (locked yes) (layer "F.Cu") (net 13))
 (segment (start 115.425 89.3) (end 115.6 90.65) (width 0.25) (locked yes) (layer "F.Cu") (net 13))
 (segment (start 69.66 92.8) (end 69.66 91.8) (width 0.25) (locked yes) (layer "F.Cu") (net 3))
 (segment (start 98.73 99.5) (end 70.8 99.5) (width 0.25) (locked yes) (layer "F.Cu") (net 3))
 (segment (start 98.73 95.4) (end 98.73 99.5) (width 0.25) (locked yes) (layer "F.Cu") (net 3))
 (segment (start 70.8 99.5) (end 70.8 91.8) (width 0.25) (locked yes) (layer "F.Cu") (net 3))
 (segment (start 75.15 87.85) (end 96 87.85) (width 0.25) (locked yes) (layer "F.Cu") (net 15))
 (segment (start 75.15 88.6) (end 75.15 87.85) (width 0.25) (locked yes) (layer "F.Cu") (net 15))
 (segment (start 96 87.85) (end 96 91.8) (width 0.25) (locked yes) (layer "F.Cu") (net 15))
 (segment (start 96 91.8) (end 97.45 91.8) (width 0.25) (locked yes) (layer "F.Cu") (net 15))
 (segment (start 123.55 91.8) (end 124.85 91.8) (width 0.25) (locked yes) (layer "F.Cu") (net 11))
 (segment (start 102.55 88.6) (end 102.55 87.85) (width 0.25) (locked yes) (layer "F.Cu") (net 11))
 (segment (start 102.55 87.85) (end 123.55 87.85) (width 0.25) (locked yes) (layer "F.Cu") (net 11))
 (segment (start 123.55 87.85) (end 123.55 91.8) (width 0.25) (locked yes) (layer "F.Cu") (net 11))
 (segment (start 68.175 91.6) (end 68.175 88.5) (width 0.25) (locked yes) (layer "F.Cu") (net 14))
 (segment (start 115.6 92.75) (end 116.5 92.75) (width 0.25) (locked yes) (layer "F.Cu") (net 14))
 (segment (start 113.8 92.525) (end 115.6 92.75) (width 0.25) (locked yes) (layer "F.Cu") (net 14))
 (segment (start 131.824999 91.6) (end 131.824999 88.5) (width 0.25) (locked yes) (layer "F.Cu") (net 14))
 (segment (start 131.824999 88.5) (end 140.165 88.5) (width 0.25) (locked yes) (layer "F.Cu") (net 14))
 (segment (start 108.89 95.4) (end 108.89 91.6) (width 0.25) (locked yes) (layer "F.Cu") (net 14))
 (segment (start 116.5 92.75) (end 116.5 91.6) (width 0.25) (locked yes) (layer "F.Cu") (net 14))
 (segment (start 68.175 88.5) (end 59.835 88.5) (width 0.25) (locked yes) (layer "F.Cu") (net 14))
 (via (at 108.89 91.6) (size 0.6) (drill 0.3) (layers "F.Cu" "B.Cu") (locked yes) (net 14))
 (via (at 68.175 91.6) (size 0.6) (drill 0.3) (layers "F.Cu" "B.Cu") (locked yes) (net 14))
 (via (at 131.824999 91.6) (size 0.6) (drill 0.3) (layers "F.Cu" "B.Cu") (locked yes) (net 14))
 (via (at 116.5 91.6) (size 0.6) (drill 0.3) (layers "F.Cu" "B.Cu") (locked yes) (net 14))
 (segment (start 68.175 91.6) (end 131.824999 91.6) (width 0.25) (locked yes) (layer "B.Cu") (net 14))
 (segment (start 107.62 94.3) (end 107.62 89.3) (width 0.25) (locked yes) (layer "F.Cu") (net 10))
 (segment (start 107.62 89.3) (end 113.775 89.3) (width 0.25) (locked yes) (layer "F.Cu") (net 10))
 (via (at 107.62 94.3) (size 0.6) (drill 0.3) (layers "F.Cu" "B.Cu") (locked yes) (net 10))
 (segment (start 101.27 95.4) (end 101.27 98.4) (width 0.25) (locked yes) (layer "F.Cu") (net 1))
 (segment (start 112.9 98.4) (end 114.6 98.4) (width 0.25) (locked yes) (layer "F.Cu") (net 1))
 (segment (start 112.9 98.4) (end 112.9 94.3) (width 0.25) (locked yes) (layer "F.Cu") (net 1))
 (segment (start 101.27 98.4) (end 112.9 98.4) (width 0.25) (locked yes) (layer "F.Cu") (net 1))
 (via (at 112.9 94.3) (size 0.6) (drill 0.3) (layers "F.Cu" "B.Cu") (locked yes) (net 1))
 (segment (start 122.1 94.3) (end 122.1 89.4) (width 1) (locked yes) (layer "F.Cu") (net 5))
 (segment (start 91.11 95.4) (end 91.11 97.95) (width 0.3) (locked yes) (layer "F.Cu") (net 5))
 (segment (start 77.5 94.3) (end 77.5 89.4) (width 1.4) (locked yes) (layer "F.Cu") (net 5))
 (segment (start 79.6 90.45) (end 79.6 89) (width 0.5) (locked yes) (layer "F.Cu") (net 5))
 (segment (start 84.6 89.625) (end 84.6 88.65) (width 0.4) (locked yes) (layer "F.Cu") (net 5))
 (segment (start 91.11 95.4) (end 91.11 89) (width 0.5) (locked yes) (layer "F.Cu") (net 5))
 (segment (start 86.775 94.3) (end 86.775 89.4) (width 1) (locked yes) (layer "F.Cu") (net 5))
 (segment (start 124.85 88.6) (end 126.6 88.6) (width 0.4) (locked yes) (layer "F.Cu") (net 5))
 (segment (start 97.45 88.6) (end 99.2 88.6) (width 0.4) (locked yes) (layer "F.Cu") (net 5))
 (segment (start 119.8 89.625) (end 119.8 88.65) (width 0.4) (locked yes) (layer "F.Cu") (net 5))
 (segment (start 105.4 89.625) (end 105.4 88.65) (width 0.4) (locked yes) (layer "F.Cu") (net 5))
 (segment (start 86.775 97.95) (end 86.775 94.3) (width 0.3) (locked yes) (layer "F.Cu") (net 5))
 (segment (start 91.11 97.95) (end 86.775 97.95) (width 0.3) (locked yes) (layer "F.Cu") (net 5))
 (segment (start 70.05 88.6) (end 71.8 88.6) (width 0.4) (locked yes) (layer "F.Cu") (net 5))
 (via (at 126.6 88.6) (size 0.6) (drill 0.3) (layers "F.Cu" "B.Cu") (locked yes) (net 5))
 (via (at 122.5 94.3) (size 0.6) (drill 0.3) (layers "F.Cu" "B.Cu") (locked yes) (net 5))
 (via (at 77.5 94.3) (size 0.6) (drill 0.3) (layers "F.Cu" "B.Cu") (locked yes) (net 5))
 (via (at 77.5 89) (size 0.6) (drill 0.3) (layers "F.Cu" "B.Cu") (locked yes) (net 5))
 (via (at 79.6 89) (size 0.6) (drill 0.3) (layers "F.Cu" "B.Cu") (locked yes) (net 5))
 (via (at 87.15 89) (size 0.6) (drill 0.3) (layers "F.Cu" "B.Cu") (locked yes) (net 5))
 (via (at 91.11 89) (size 0.6) (drill 0.3) (layers "F.Cu" "B.Cu") (locked yes) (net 5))
 (via (at 121.7 89) (size 0.6) (drill 0.3) (layers "F.Cu" "B.Cu") (locked yes) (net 5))
 (via (at 121.7 94.3) (size 0.6) (drill 0.3) (layers "F.Cu" "B.Cu") (locked yes) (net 5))
 (via (at 76.7 89) (size 0.6) (drill 0.3) (layers "F.Cu" "B.Cu") (locked yes) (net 5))
 (via (at 78.3 89) (size 0.6) (drill 0.3) (layers "F.Cu" "B.Cu") (locked yes) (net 5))
 (via (at 87.15 94.3) (size 0.6) (drill 0.3) (layers "F.Cu" "B.Cu") (locked yes) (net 5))
 (via (at 105.4 88.65) (size 0.6) (drill 0.3) (layers "F.Cu" "B.Cu") (locked yes) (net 5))
 (via (at 86.4 94.3) (size 0.6) (drill 0.3) (layers "F.Cu" "B.Cu") (locked yes) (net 5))
 (via (at 76.7 94.3) (size 0.6) (drill 0.3) (layers "F.Cu" "B.Cu") (locked yes) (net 5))
 (via (at 99.2 88.6) (size 0.6) (drill 0.3) (layers "F.Cu" "B.Cu") (locked yes) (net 5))
 (via (at 71.8 88.6) (size 0.6) (drill 0.3) (layers "F.Cu" "B.Cu") (locked yes) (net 5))
 (via (at 86.4 89) (size 0.6) (drill 0.3) (layers "F.Cu" "B.Cu") (locked yes) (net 5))
 (via (at 119.8 88.65) (size 0.6) (drill 0.3) (layers "F.Cu" "B.Cu") (locked yes) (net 5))
 (via (at 78.3 94.3) (size 0.6) (drill 0.3) (layers "F.Cu" "B.Cu") (locked yes) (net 5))
 (via (at 122.5 89) (size 0.6) (drill 0.3) (layers "F.Cu" "B.Cu") (locked yes) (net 5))
 (via (at 84.6 88.65) (size 0.6) (drill 0.3) (layers "F.Cu" "B.Cu") (locked yes) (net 5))
 (segment (start 136.825 88.6) (end 136.825 92.75) (width 1.2) (locked yes) (layer "B.Cu") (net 5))
 (segment (start 136.825 92.75) (end 139.665 92.75) (width 1.2) (locked yes) (layer "B.Cu") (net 5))
 (segment (start 63.175 92.75) (end 60.335 92.75) (width 1.2) (locked yes) (layer "B.Cu") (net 5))
 (segment (start 63.175 88.6) (end 136.825 88.6) (width 1.4) (locked yes) (layer "B.Cu") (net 5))
 (segment (start 63.175 88.6) (end 63.175 92.75) (width 1.2) (locked yes) (layer "B.Cu") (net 5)))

